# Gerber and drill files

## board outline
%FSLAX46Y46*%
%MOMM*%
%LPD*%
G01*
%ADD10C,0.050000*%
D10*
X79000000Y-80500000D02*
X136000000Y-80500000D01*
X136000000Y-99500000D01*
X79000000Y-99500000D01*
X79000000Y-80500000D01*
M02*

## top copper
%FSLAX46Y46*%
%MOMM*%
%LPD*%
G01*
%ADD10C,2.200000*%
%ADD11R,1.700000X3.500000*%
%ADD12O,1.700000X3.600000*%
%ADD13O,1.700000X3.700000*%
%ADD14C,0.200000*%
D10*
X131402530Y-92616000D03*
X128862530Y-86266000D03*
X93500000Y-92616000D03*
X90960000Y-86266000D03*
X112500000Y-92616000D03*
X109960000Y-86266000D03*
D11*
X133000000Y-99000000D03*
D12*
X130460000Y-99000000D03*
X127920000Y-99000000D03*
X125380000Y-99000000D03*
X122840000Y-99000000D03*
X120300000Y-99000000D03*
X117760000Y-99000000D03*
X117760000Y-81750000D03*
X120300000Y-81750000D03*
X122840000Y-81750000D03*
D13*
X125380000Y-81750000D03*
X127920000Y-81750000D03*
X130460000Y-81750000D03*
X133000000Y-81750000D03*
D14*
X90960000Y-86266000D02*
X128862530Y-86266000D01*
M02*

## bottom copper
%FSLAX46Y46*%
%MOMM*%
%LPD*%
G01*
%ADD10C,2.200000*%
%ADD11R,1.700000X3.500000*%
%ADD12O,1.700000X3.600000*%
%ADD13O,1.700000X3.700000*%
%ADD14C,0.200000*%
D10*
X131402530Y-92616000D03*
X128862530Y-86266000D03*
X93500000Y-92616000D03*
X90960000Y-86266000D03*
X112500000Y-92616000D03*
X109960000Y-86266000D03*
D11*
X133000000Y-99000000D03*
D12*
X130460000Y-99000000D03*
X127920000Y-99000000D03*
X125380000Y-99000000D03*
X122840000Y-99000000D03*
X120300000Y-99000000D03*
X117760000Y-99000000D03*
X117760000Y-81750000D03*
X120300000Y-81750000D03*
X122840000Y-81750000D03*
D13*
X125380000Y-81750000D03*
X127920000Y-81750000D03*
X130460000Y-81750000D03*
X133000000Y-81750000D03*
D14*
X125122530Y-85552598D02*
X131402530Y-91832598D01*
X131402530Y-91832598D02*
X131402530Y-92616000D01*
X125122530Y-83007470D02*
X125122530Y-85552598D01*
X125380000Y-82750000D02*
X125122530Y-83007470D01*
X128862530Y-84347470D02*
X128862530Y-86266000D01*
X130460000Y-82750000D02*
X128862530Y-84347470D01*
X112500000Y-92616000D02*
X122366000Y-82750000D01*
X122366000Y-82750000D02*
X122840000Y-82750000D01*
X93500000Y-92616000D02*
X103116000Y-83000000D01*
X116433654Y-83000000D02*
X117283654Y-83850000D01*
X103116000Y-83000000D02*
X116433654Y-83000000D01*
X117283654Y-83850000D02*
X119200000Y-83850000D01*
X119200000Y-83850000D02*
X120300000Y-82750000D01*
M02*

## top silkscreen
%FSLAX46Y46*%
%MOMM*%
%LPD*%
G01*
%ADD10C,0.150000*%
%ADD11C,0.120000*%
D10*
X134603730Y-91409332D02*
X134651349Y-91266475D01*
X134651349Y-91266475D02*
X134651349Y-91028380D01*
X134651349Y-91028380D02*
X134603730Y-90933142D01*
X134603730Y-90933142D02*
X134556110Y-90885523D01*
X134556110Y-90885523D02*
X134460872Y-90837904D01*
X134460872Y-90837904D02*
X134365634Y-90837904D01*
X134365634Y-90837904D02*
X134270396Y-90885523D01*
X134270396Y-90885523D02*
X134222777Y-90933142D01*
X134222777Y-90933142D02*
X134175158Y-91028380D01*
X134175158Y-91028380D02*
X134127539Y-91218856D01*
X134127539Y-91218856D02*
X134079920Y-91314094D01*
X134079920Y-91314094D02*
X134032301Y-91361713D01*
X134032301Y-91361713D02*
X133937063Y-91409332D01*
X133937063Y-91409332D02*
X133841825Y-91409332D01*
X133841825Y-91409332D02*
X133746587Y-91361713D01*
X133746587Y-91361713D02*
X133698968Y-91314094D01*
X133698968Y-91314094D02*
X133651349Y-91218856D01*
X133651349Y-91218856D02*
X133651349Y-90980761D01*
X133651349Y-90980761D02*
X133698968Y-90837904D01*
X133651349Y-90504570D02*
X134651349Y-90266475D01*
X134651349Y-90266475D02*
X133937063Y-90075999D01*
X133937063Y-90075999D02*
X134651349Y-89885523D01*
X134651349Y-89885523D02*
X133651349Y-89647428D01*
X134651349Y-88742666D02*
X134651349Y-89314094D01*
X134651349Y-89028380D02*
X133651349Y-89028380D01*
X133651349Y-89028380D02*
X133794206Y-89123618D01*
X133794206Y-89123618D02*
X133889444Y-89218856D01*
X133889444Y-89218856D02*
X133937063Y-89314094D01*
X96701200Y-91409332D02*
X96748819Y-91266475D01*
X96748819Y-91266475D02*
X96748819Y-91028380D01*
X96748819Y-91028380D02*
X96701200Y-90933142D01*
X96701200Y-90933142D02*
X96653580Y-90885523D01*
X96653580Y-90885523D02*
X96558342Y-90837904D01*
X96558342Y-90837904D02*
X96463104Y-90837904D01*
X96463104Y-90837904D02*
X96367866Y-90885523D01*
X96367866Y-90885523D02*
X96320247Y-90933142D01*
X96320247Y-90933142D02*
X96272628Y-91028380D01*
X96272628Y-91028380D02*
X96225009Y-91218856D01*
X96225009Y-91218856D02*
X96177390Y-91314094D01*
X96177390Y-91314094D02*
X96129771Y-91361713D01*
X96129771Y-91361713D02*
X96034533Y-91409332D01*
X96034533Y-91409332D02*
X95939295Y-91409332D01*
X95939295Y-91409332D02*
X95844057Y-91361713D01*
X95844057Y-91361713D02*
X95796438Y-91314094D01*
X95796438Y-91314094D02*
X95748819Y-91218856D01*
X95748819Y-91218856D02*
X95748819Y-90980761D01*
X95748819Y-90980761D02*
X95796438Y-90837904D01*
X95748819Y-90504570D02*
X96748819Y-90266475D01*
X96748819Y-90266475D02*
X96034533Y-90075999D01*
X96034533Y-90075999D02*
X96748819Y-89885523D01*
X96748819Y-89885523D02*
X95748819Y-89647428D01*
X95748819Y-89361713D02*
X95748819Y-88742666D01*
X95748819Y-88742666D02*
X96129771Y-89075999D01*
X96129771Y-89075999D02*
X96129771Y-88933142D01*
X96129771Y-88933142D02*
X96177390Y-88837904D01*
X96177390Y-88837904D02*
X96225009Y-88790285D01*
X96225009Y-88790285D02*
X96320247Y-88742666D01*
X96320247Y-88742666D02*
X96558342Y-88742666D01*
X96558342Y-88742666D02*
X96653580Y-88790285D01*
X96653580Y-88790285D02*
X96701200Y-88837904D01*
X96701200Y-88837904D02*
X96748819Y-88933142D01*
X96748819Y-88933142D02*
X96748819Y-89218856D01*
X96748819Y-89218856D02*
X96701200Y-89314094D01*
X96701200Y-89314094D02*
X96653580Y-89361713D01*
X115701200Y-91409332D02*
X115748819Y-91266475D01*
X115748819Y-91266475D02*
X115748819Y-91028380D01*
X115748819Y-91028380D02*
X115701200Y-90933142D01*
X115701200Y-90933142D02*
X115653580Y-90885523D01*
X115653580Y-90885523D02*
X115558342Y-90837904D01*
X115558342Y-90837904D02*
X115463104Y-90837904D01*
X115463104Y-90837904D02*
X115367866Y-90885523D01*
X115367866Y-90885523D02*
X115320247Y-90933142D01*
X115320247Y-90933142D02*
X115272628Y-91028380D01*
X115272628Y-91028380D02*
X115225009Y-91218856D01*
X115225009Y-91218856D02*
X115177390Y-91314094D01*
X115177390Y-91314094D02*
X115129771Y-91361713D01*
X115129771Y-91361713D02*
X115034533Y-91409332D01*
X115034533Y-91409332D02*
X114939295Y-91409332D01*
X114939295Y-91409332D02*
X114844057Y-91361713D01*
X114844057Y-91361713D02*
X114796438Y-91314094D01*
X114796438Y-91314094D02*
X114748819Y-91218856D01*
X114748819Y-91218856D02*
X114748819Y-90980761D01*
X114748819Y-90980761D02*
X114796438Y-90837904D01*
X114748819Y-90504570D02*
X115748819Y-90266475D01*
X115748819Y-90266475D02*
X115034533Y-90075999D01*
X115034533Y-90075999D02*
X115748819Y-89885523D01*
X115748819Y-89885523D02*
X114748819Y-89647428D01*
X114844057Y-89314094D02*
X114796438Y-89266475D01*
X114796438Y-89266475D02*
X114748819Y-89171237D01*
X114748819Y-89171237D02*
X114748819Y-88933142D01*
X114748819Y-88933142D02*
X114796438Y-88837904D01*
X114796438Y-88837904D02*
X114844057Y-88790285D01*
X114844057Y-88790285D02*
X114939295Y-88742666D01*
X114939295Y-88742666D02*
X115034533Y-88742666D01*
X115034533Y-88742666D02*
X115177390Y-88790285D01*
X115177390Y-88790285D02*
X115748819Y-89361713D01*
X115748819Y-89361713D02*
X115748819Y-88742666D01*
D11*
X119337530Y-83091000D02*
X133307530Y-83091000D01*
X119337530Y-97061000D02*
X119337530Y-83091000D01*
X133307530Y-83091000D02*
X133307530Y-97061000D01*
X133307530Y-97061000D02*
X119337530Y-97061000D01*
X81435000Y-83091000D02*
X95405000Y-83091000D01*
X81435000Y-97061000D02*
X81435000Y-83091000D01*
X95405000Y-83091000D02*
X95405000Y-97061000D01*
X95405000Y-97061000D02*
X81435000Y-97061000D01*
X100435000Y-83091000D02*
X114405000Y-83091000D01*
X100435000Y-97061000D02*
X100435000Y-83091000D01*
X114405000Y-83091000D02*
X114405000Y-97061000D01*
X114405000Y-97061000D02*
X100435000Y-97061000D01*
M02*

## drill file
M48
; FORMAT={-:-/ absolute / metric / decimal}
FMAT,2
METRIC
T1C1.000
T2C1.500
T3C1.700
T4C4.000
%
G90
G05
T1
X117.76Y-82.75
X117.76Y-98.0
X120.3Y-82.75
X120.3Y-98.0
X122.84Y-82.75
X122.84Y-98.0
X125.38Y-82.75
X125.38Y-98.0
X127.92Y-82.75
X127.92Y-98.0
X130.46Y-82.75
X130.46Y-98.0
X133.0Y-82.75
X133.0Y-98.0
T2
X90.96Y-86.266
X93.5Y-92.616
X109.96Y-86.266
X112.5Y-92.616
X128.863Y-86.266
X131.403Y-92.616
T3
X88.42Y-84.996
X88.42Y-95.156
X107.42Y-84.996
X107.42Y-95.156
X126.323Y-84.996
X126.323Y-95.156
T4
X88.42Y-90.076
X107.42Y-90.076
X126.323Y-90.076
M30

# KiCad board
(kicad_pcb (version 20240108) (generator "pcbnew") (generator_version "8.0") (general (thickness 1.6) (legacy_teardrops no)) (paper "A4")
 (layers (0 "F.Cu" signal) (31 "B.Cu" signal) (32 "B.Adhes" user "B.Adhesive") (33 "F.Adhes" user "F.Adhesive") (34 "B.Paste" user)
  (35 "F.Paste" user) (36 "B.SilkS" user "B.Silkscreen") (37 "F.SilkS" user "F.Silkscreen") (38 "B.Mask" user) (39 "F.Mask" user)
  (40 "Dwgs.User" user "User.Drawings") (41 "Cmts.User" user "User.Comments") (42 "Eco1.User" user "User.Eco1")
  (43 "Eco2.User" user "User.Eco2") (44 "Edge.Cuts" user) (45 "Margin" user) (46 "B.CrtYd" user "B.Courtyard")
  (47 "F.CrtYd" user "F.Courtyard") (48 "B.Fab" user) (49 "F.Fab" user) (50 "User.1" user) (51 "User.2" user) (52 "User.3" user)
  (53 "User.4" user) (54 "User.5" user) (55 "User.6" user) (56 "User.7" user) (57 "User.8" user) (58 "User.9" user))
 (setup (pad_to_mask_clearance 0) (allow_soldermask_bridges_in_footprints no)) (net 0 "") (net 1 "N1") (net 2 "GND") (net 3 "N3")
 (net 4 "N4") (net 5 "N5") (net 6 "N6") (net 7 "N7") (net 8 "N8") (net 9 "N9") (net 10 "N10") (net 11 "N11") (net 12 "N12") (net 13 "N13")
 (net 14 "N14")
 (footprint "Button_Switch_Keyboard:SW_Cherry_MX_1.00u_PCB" (layer "F.Cu") (at 131.40253 92.616 -90)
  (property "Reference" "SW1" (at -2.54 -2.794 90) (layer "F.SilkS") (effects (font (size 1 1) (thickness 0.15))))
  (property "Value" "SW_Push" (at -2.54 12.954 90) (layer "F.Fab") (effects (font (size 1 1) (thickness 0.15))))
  (fp_line (start -9.525 12.065) (end -9.525 -1.905) (stroke (width 0.12) (type solid)) (layer "F.SilkS"))
  (fp_line (start 4.445 12.065) (end -9.525 12.065) (stroke (width 0.12) (type solid)) (layer "F.SilkS"))
  (fp_line (start -9.525 -1.905) (end 4.445 -1.905) (stroke (width 0.12) (type solid)) (layer "F.SilkS"))
  (fp_line (start 4.445 -1.905) (end 4.445 12.065) (stroke (width 0.12) (type solid)) (layer "F.SilkS"))
  (pad "" np_thru_hole circle (at -7.62 5.08 270) (size 1.7 1.7) (drill 1.7) (layers "*.Cu" "*.Mask"))
  (pad "" np_thru_hole circle (at -2.54 5.08 270) (size 4 4) (drill 4) (layers "*.Cu" "*.Mask"))
  (pad "" np_thru_hole circle (at 2.54 5.08 270) (size 1.7 1.7) (drill 1.7) (layers "*.Cu" "*.Mask"))
  (pad "1" thru_hole circle (at 0 0 270) (size 2.2 2.2) (drill 1.5) (layers "*.Cu" "*.Mask") (remove_unused_layers no) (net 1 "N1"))
  (pad "2" thru_hole circle (at -6.35 2.54 270) (size 2.2 2.2) (drill 1.5) (layers "*.Cu" "*.Mask") (remove_unused_layers no) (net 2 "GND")))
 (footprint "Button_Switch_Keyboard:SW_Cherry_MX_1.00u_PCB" (layer "F.Cu") (at 93.5 92.616 -90)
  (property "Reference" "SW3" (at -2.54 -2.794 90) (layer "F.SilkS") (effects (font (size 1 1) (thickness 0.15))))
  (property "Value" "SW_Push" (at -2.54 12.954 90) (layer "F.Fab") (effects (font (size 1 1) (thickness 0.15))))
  (fp_line (start -9.525 12.065) (end -9.525 -1.905) (stroke (width 0.12) (type solid)) (layer "F.SilkS"))
  (fp_line (start 4.445 12.065) (end -9.525 12.065) (stroke (width 0.12) (type solid)) (layer "F.SilkS"))
  (fp_line (start -9.525 -1.905) (end 4.445 -1.905) (stroke (width 0.12) (type solid)) (layer "F.SilkS"))
  (fp_line (start 4.445 -1.905) (end 4.445 12.065) (stroke (width 0.12) (type solid)) (layer "F.SilkS"))
  (pad "" np_thru_hole circle (at -7.62 5.08 270) (size 1.7 1.7) (drill 1.7) (layers "*.Cu" "*.Mask"))
  (pad "" np_thru_hole circle (at -2.54 5.08 270) (size 4 4) (drill 4) (layers "*.Cu" "*.Mask"))
  (pad "" np_thru_hole circle (at 2.54 5.08 270) (size 1.7 1.7) (drill 1.7) (layers "*.Cu" "*.Mask"))
  (pad "1" thru_hole circle (at 0 0 270) (size 2.2 2.2) (drill 1.5) (layers "*.Cu" "*.Mask") (remove_unused_layers no) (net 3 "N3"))
  (pad "2" thru_hole circle (at -6.35 2.54 270) (size 2.2 2.2) (drill 1.5) (layers "*.Cu" "*.Mask") (remove_unused_layers no) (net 2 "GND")))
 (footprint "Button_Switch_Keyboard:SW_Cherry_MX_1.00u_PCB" (layer "F.Cu") (at 112.5 92.616 -90)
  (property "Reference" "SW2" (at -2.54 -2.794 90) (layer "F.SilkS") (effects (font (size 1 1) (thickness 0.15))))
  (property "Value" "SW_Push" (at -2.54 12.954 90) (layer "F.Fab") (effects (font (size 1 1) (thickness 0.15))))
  (fp_line (start -9.525 12.065) (end -9.525 -1.905) (stroke (width 0.12) (type solid)) (layer "F.SilkS"))
  (fp_line (start 4.445 12.065) (end -9.525 12.065) (stroke (width 0.12) (type solid)) (layer "F.SilkS"))
  (fp_line (start -9.525 -1.905) (end 4.445 -1.905) (stroke (width 0.12) (type solid)) (layer "F.SilkS"))
  (fp_line (start 4.445 -1.905) (end 4.445 12.065) (stroke (width 0.12) (type solid)) (layer "F.SilkS"))
  (pad "" np_thru_hole circle (at -7.62 5.08 270) (size 1.7 1.7) (drill 1.7) (layers "*.Cu" "*.Mask"))
  (pad "" np_thru_hole circle (at -2.54 5.08 270) (size 4 4) (drill 4) (layers "*.Cu" "*.Mask"))
  (pad "" np_thru_hole circle (at 2.54 5.08 270) (size 1.7 1.7) (drill 1.7) (layers "*.Cu" "*.Mask"))
  (pad "1" thru_hole circle (at 0 0 270) (size 2.2 2.2) (drill 1.5) (layers "*.Cu" "*.Mask") (remove_unused_layers no) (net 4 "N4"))
  (pad "2" thru_hole circle (at -6.35 2.54 270) (size 2.2 2.2) (drill 1.5) (layers "*.Cu" "*.Mask") (remove_unused_layers no) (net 2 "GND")))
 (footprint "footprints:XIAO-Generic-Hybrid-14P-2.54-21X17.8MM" (layer "B.Cu") (at 125.38 90.375 90)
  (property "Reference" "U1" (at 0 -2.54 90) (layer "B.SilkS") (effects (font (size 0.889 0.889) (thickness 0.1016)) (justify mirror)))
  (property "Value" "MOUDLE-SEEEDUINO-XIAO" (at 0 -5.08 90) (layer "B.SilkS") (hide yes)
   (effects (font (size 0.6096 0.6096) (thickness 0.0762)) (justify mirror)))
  (pad "1" thru_hole rect (at -7.625 7.62 90) (size 3.5 1.7) (drill 1 (offset -1 0)) (layers "*.Cu" "*.Mask") (remove_unused_layers no)
   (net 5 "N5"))
  (pad "2" thru_hole oval (at -7.625 5.08 90) (size 3.6 1.7) (drill 1 (offset -1 0)) (layers "*.Cu" "*.Mask") (remove_unused_layers no)
   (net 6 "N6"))
  (pad "3" thru_hole oval (at -7.625 2.54 90) (size 3.6 1.7) (drill 1 (offset -1 0)) (layers "*.Cu" "*.Mask") (remove_unused_layers no)
   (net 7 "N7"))
  (pad "4" thru_hole oval (at -7.625 0 90) (size 3.6 1.7) (drill 1 (offset -1 0)) (layers "*.Cu" "*.Mask") (remove_unused_layers no)
   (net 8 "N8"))
  (pad "5" thru_hole oval (at -7.625 -2.54 90) (size 3.6 1.7) (drill 1 (offset -1 0)) (layers "*.Cu" "*.Mask") (remove_unused_layers no)
   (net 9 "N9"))
  (pad "6" thru_hole oval (at -7.625 -5.08 270) (size 3.6 1.7) (drill 1 (offset 1 0)) (layers "*.Cu" "*.Mask") (remove_unused_layers no)
   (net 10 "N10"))
  (pad "7" thru_hole oval (at -7.625 -7.62 90) (size 3.6 1.7) (drill 1 (offset -1 0)) (layers "*.Cu" "*.Mask") (remove_unused_layers no)
   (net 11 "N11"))
  (pad "8" thru_hole oval (at 7.625 -7.62 90) (size 3.6 1.7) (drill 1 (offset 1 0)) (layers "*.Cu" "*.Mask") (remove_unused_layers no)
   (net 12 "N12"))
  (pad "9" thru_hole oval (at 7.625 -5.08 90) (size 3.6 1.7) (drill 1 (offset 1 0)) (layers "*.Cu" "*.Mask") (remove_unused_layers no)
   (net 3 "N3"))
  (pad "10" thru_hole oval (at 7.625 -2.54 90) (size 3.6 1.7) (drill 1 (offset 1 0)) (layers "*.Cu" "*.Mask") (remove_unused_layers no)
   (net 4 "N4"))
  (pad "11" thru_hole oval (at 7.625 0 90) (size 3.7 1.7) (drill 1 (offset 1 0)) (layers "*.Cu" "*.Mask") (remove_unused_layers no)
   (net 1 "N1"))
  (pad "12" thru_hole oval (at 7.625 2.54 90) (size 3.7 1.7) (drill 1 (offset 1 0)) (layers "*.Cu" "*.Mask") (remove_unused_layers no)
   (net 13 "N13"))
  (pad "13" thru_hole oval (at 7.625 5.08 90) (size 3.7 1.7) (drill 1 (offset 1 0)) (layers "*.Cu" "*.Mask") (remove_unused_layers no)
   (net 2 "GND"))
  (pad "14" thru_hole oval (at 7.625 7.62 90) (size 3.7 1.7) (drill 1 (offset 1 0)) (layers "*.Cu" "*.Mask") (remove_unused_layers no)
   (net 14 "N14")))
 (gr_rect (start 79 80.5) (end 136 99.5) (stroke (width 0.05) (type default)) (fill none) (layer "Edge.Cuts"))
 (segment (start 125.12253 85.552598) (end 131.40253 91.832598) (width 0.2) (layer "B.Cu") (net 1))
 (segment (start 131.40253 91.832598) (end 131.40253 92.616) (width 0.2) (layer "B.Cu") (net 1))
 (segment (start 125.12253 83.00747) (end 125.12253 85.552598) (width 0.2) (layer "B.Cu") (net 1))
 (segment (start 125.38 82.75) (end 125.12253 83.00747) (width 0.2) (layer "B.Cu") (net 1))
 (segment (start 90.96 86.266) (end 128.86253 86.266) (width 0.2) (layer "F.Cu") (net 2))
 (segment (start 128.86253 84.34747) (end 128.86253 86.266) (width 0.2) (layer "B.Cu") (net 2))
 (segment (start 130.46 82.75) (end 128.86253 84.34747) (width 0.2) (layer "B.Cu") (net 2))
 (segment (start 112.5 92.616) (end 122.366 82.75) (width 0.2) (layer "B.Cu") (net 4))
 (segment (start 122.366 82.75) (end 122.84 82.75) (width 0.2) (layer "B.Cu") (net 4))
 (segment (start 93.5 92.616) (end 103.116 83) (width 0.2) (layer "B.Cu") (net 3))
 (segment (start 116.433654 83) (end 117.283654 83.85) (width 0.2) (layer "B.Cu") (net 3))
 (segment (start 103.116 83) (end 116.433654 83) (width 0.2) (layer "B.Cu") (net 3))
 (segment (start 117.283654 83.85) (end 119.2 83.85) (width 0.2) (layer "B.Cu") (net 3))
 (segment (start 119.2 83.85) (end 120.3 82.75) (width 0.2) (layer "B.Cu") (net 3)))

